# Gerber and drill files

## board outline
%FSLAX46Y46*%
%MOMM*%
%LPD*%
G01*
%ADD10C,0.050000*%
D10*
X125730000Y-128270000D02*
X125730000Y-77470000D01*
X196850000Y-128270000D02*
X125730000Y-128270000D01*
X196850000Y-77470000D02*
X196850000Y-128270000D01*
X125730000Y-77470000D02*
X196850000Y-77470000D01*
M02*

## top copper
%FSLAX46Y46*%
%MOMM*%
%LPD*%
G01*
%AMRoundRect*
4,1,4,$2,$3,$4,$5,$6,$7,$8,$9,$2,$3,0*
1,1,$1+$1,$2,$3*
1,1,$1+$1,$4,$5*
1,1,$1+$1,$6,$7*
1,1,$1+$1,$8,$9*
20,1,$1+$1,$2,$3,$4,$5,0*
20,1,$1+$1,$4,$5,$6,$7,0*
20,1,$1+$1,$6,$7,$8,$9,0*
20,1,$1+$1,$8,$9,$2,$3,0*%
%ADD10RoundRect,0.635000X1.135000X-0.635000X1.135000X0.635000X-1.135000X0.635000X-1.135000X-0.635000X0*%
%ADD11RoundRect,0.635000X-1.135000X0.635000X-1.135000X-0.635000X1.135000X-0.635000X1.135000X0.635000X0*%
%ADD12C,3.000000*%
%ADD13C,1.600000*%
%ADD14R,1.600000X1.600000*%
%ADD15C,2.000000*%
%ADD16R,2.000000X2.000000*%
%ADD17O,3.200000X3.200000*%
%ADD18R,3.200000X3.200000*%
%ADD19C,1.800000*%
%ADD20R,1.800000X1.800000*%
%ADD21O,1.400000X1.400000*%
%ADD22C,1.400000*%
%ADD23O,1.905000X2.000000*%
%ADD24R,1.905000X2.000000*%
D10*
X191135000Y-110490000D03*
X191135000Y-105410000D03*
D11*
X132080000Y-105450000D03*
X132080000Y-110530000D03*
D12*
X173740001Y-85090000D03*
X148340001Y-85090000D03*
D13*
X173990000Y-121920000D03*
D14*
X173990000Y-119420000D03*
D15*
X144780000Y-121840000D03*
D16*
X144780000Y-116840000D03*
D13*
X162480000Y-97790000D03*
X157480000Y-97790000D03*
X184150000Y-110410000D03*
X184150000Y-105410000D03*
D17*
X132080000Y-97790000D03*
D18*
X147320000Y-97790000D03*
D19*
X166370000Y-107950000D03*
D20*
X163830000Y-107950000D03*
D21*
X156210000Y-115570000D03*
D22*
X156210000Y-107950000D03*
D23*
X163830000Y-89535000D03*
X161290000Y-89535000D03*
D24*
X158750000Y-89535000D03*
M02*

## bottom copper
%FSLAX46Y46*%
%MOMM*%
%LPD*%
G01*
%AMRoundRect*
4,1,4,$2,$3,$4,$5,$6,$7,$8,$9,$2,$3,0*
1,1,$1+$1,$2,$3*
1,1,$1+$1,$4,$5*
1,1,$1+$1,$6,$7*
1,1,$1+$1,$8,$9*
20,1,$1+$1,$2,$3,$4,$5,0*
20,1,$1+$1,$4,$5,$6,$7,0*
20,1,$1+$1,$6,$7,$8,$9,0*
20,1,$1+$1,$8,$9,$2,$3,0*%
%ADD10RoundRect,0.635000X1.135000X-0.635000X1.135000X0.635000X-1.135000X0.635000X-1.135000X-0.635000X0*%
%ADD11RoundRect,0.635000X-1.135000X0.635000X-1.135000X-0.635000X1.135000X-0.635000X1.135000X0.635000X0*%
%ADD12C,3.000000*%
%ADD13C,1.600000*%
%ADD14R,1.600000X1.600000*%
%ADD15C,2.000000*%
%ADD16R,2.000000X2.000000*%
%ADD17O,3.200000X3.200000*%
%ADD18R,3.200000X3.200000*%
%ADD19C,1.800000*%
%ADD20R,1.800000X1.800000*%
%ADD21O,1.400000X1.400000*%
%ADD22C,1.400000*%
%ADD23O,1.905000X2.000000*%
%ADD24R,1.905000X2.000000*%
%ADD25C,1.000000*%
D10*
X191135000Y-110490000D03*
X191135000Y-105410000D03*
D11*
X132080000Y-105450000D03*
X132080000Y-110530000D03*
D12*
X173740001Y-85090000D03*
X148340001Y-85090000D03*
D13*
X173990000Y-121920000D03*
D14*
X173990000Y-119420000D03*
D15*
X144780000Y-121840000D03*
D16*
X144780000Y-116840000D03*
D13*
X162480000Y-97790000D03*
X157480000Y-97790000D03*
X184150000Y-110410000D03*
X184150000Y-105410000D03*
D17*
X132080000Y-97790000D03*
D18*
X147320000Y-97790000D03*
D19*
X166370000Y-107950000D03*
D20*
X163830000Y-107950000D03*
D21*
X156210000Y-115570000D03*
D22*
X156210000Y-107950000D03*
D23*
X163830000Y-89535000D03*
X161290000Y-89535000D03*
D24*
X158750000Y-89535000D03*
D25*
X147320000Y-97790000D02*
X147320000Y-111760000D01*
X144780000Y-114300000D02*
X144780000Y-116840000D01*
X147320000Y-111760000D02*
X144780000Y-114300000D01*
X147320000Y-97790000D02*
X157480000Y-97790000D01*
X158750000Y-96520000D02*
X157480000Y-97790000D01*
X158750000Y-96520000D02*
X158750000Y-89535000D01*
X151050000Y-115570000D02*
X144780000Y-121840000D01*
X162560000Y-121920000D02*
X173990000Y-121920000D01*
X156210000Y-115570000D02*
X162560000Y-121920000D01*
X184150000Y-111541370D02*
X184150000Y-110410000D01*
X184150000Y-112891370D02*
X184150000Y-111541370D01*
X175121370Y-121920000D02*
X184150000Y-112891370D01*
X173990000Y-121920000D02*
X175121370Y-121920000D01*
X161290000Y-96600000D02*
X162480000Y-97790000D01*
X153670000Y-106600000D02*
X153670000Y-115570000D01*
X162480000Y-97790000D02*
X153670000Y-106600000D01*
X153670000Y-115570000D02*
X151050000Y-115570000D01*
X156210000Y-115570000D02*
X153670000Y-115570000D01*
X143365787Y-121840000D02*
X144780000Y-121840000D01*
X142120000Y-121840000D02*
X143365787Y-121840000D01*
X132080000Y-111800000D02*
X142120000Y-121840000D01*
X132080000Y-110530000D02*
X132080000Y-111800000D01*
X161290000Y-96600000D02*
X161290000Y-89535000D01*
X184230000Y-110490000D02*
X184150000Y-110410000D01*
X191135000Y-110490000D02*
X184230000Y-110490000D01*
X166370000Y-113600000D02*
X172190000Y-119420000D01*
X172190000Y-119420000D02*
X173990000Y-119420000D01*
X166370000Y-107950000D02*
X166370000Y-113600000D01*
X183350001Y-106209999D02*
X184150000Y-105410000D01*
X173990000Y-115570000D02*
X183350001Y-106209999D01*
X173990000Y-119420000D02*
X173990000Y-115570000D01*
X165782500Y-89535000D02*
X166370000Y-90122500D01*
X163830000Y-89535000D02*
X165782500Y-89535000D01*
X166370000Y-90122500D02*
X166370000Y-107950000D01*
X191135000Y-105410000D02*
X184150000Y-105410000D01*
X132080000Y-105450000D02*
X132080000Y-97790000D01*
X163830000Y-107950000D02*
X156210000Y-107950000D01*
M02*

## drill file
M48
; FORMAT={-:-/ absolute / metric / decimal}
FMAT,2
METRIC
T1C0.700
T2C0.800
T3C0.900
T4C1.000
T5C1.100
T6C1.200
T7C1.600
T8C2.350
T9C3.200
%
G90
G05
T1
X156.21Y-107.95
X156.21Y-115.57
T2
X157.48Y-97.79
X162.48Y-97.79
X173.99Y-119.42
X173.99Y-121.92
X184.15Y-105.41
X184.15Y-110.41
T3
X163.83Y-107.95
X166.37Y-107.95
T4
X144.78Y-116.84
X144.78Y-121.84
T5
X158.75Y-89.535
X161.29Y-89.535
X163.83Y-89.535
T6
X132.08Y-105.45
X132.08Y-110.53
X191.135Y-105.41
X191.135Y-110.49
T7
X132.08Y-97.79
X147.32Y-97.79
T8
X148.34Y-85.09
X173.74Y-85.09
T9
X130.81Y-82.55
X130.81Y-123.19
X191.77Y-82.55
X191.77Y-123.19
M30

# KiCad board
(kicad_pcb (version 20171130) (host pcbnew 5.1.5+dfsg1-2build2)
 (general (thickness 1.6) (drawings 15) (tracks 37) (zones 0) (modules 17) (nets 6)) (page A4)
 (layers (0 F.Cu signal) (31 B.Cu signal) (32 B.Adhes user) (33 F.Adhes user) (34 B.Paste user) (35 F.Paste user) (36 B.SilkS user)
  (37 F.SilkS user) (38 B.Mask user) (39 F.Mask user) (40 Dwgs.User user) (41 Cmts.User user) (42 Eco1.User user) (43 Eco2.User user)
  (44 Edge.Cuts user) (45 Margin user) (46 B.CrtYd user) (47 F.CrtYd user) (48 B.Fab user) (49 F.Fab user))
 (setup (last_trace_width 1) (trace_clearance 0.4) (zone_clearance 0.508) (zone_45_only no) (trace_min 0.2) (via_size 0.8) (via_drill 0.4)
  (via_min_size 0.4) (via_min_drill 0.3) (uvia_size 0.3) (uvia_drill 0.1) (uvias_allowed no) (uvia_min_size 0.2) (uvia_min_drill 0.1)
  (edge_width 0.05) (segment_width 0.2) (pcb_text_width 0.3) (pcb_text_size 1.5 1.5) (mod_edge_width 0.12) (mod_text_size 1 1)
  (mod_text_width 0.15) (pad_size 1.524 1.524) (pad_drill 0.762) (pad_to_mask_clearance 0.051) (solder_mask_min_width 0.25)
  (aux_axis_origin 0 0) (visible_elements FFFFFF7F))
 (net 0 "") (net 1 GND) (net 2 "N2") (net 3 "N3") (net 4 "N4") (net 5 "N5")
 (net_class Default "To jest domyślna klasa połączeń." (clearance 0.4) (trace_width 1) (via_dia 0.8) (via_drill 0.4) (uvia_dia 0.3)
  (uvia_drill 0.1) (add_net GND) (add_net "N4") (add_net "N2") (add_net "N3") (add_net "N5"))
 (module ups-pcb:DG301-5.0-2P (layer F.Cu) (at 191.135 107.99 90)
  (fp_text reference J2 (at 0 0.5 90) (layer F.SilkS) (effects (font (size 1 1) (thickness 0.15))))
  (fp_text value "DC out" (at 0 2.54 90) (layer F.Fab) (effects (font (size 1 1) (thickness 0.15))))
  (pad 1 thru_hole roundrect (at -2.5 0 90) (size 2.54 3.54) (drill 1.2) (layers *.Cu *.Mask) (roundrect_rratio 0.25) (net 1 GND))
  (pad 2 thru_hole roundrect (at 2.58 0 90) (size 2.54 3.54) (drill 1.2) (layers *.Cu *.Mask) (roundrect_rratio 0.25) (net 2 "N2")))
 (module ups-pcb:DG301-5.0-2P (layer F.Cu) (at 132.08 107.95 270)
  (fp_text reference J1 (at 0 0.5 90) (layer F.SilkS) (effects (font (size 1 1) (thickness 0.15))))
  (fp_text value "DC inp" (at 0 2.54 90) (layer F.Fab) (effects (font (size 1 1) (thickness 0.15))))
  (pad 1 thru_hole roundrect (at -2.5 0 270) (size 2.54 3.54) (drill 1.2) (layers *.Cu *.Mask) (roundrect_rratio 0.25) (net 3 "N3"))
  (pad 2 thru_hole roundrect (at 2.58 0 270) (size 2.54 3.54) (drill 1.2) (layers *.Cu *.Mask) (roundrect_rratio 0.25) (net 1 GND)))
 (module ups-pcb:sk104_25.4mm (layer F.Cu) (at 161.040001 85.09)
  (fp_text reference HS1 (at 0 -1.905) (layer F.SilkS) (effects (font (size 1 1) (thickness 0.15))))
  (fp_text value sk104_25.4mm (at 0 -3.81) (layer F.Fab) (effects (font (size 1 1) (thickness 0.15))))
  (pad "" np_thru_hole circle (at 12.7 0) (size 3 3) (drill 2.35) (layers *.Cu *.Mask))
  (pad "" np_thru_hole circle (at -12.7 0) (size 3 3) (drill 2.35) (layers *.Cu *.Mask)))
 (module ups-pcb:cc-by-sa (layer F.Cu) (at 159.385 121.92)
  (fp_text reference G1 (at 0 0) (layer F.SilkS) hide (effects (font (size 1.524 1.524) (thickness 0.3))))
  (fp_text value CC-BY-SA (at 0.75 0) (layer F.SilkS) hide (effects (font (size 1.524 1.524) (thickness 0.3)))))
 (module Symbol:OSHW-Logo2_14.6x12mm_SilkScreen (layer F.Cu) (at 186.055 93.98)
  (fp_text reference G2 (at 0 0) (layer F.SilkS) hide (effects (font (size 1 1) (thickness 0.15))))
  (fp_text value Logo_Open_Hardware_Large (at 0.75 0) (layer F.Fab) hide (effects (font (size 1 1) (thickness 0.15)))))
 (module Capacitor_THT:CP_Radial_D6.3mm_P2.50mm (layer F.Cu) (at 173.99 119.42 270)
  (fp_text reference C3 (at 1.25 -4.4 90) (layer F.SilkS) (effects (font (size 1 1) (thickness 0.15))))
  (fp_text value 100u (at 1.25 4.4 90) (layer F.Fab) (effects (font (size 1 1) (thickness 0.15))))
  (pad 2 thru_hole circle (at 2.5 0 270) (size 1.6 1.6) (drill 0.8) (layers *.Cu *.Mask) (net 1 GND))
  (pad 1 thru_hole rect (at 0 0 270) (size 1.6 1.6) (drill 0.8) (layers *.Cu *.Mask) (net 2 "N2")))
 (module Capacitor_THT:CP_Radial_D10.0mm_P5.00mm (layer F.Cu) (at 144.78 116.84 270)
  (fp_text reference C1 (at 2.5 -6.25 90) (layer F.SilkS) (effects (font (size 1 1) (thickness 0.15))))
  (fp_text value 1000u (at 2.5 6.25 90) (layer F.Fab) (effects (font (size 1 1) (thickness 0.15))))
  (pad 2 thru_hole circle (at 5 0 270) (size 2 2) (drill 1) (layers *.Cu *.Mask) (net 1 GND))
  (pad 1 thru_hole rect (at 0 0 270) (size 2 2) (drill 1) (layers *.Cu *.Mask) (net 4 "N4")))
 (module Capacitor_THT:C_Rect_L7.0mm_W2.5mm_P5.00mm (layer F.Cu) (at 157.48 97.79)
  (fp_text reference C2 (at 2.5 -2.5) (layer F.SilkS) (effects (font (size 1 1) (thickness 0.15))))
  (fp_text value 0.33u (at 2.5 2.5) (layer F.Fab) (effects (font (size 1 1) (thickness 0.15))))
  (pad 2 thru_hole circle (at 5 0) (size 1.6 1.6) (drill 0.8) (layers *.Cu *.Mask) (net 1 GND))
  (pad 1 thru_hole circle (at 0 0) (size 1.6 1.6) (drill 0.8) (layers *.Cu *.Mask) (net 4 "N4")))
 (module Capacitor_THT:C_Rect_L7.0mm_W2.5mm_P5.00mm (layer F.Cu) (at 184.15 105.41 270)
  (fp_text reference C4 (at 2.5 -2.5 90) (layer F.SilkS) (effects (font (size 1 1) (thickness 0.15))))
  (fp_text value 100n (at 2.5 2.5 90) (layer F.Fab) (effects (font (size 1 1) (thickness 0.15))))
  (pad 2 thru_hole circle (at 5 0 270) (size 1.6 1.6) (drill 0.8) (layers *.Cu *.Mask) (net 1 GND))
  (pad 1 thru_hole circle (at 0 0 270) (size 1.6 1.6) (drill 0.8) (layers *.Cu *.Mask) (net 2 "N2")))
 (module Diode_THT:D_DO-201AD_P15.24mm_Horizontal (layer F.Cu) (at 147.32 97.79 180)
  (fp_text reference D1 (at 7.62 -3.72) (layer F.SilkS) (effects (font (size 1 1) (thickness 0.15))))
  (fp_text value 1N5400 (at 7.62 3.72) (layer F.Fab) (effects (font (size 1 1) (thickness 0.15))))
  (pad 2 thru_hole oval (at 15.24 0 180) (size 3.2 3.2) (drill 1.6) (layers *.Cu *.Mask) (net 3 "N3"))
  (pad 1 thru_hole rect (at 0 0 180) (size 3.2 3.2) (drill 1.6) (layers *.Cu *.Mask) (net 4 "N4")))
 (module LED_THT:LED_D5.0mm (layer F.Cu) (at 163.83 107.95)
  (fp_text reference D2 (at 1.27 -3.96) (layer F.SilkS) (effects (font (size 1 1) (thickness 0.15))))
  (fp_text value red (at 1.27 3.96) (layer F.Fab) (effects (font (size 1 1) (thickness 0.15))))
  (pad 2 thru_hole circle (at 2.54 0) (size 1.8 1.8) (drill 0.9) (layers *.Cu *.Mask) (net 2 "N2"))
  (pad 1 thru_hole rect (at 0 0) (size 1.8 1.8) (drill 0.9) (layers *.Cu *.Mask) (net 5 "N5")))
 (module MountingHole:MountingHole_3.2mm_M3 (layer F.Cu) (at 130.81 82.55)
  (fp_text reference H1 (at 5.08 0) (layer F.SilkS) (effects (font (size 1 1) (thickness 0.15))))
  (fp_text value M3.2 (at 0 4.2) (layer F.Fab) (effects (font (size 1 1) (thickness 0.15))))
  (pad 1 np_thru_hole circle (at 0 0) (size 3.2 3.2) (drill 3.2) (layers *.Cu *.Mask)))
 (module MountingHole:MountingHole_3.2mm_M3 (layer F.Cu) (at 191.77 82.55)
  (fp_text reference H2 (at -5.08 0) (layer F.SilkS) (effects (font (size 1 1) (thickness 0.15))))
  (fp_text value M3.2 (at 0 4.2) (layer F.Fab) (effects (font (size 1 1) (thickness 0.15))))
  (pad 1 np_thru_hole circle (at 0 0) (size 3.2 3.2) (drill 3.2) (layers *.Cu *.Mask)))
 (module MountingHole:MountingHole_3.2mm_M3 (layer F.Cu) (at 191.77 123.19)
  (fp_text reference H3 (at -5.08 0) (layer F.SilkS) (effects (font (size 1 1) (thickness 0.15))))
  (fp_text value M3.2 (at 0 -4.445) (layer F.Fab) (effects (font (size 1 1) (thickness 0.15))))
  (pad 1 np_thru_hole circle (at 0 0) (size 3.2 3.2) (drill 3.2) (layers *.Cu *.Mask)))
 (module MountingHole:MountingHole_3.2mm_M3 (layer F.Cu) (at 130.81 123.19)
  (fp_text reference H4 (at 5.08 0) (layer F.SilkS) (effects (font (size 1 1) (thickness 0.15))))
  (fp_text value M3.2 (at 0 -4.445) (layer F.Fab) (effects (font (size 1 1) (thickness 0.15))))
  (pad 1 np_thru_hole circle (at 0 0) (size 3.2 3.2) (drill 3.2) (layers *.Cu *.Mask)))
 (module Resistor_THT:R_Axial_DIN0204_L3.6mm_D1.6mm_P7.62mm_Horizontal (layer F.Cu) (at 156.21 107.95 270)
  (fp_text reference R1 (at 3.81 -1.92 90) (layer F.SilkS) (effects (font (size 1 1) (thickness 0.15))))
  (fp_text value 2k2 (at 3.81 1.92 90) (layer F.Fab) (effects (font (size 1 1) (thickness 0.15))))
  (pad 2 thru_hole oval (at 7.62 0 270) (size 1.4 1.4) (drill 0.7) (layers *.Cu *.Mask) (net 1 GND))
  (pad 1 thru_hole circle (at 0 0 270) (size 1.4 1.4) (drill 0.7) (layers *.Cu *.Mask) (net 5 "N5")))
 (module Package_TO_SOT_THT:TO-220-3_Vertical (layer F.Cu) (at 158.75 89.535)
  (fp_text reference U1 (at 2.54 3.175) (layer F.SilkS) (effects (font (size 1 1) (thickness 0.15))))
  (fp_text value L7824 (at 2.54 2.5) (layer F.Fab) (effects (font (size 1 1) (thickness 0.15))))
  (pad 3 thru_hole oval (at 5.08 0) (size 1.905 2) (drill 1.1) (layers *.Cu *.Mask) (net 2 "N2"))
  (pad 2 thru_hole oval (at 2.54 0) (size 1.905 2) (drill 1.1) (layers *.Cu *.Mask) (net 1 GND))
  (pad 1 thru_hole rect (at 0 0) (size 1.905 2) (drill 1.1) (layers *.Cu *.Mask) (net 4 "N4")))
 (gr_line (start 125.73 128.27) (end 125.73 77.47) (layer Edge.Cuts) (width 0.05))
 (gr_line (start 196.85 128.27) (end 125.73 128.27) (layer Edge.Cuts) (width 0.05))
 (gr_line (start 196.85 77.47) (end 196.85 128.27) (layer Edge.Cuts) (width 0.05))
 (gr_line (start 125.73 77.47) (end 196.85 77.47) (layer Edge.Cuts) (width 0.05))
 (segment (start 147.32 97.79) (end 147.32 111.76) (width 1) (layer B.Cu) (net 4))
 (segment (start 144.78 114.3) (end 144.78 116.84) (width 1) (layer B.Cu) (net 4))
 (segment (start 147.32 111.76) (end 144.78 114.3) (width 1) (layer B.Cu) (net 4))
 (segment (start 147.32 97.79) (end 157.48 97.79) (width 1) (layer B.Cu) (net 4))
 (segment (start 158.75 96.52) (end 157.48 97.79) (width 1) (layer B.Cu) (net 4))
 (segment (start 158.75 96.52) (end 158.75 89.535) (width 1) (layer B.Cu) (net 4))
 (segment (start 151.05 115.57) (end 144.78 121.84) (width 1) (layer B.Cu) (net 1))
 (segment (start 162.56 121.92) (end 173.99 121.92) (width 1) (layer B.Cu) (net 1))
 (segment (start 156.21 115.57) (end 162.56 121.92) (width 1) (layer B.Cu) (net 1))
 (segment (start 184.15 111.54137) (end 184.15 110.41) (width 1) (layer B.Cu) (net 1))
 (segment (start 184.15 112.89137) (end 184.15 111.54137) (width 1) (layer B.Cu) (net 1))
 (segment (start 175.12137 121.92) (end 184.15 112.89137) (width 1) (layer B.Cu) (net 1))
 (segment (start 173.99 121.92) (end 175.12137 121.92) (width 1) (layer B.Cu) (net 1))
 (segment (start 161.29 96.6) (end 162.48 97.79) (width 1) (layer B.Cu) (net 1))
 (segment (start 153.67 106.6) (end 153.67 115.57) (width 1) (layer B.Cu) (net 1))
 (segment (start 162.48 97.79) (end 153.67 106.6) (width 1) (layer B.Cu) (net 1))
 (segment (start 153.67 115.57) (end 151.05 115.57) (width 1) (layer B.Cu) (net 1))
 (segment (start 156.21 115.57) (end 153.67 115.57) (width 1) (layer B.Cu) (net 1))
 (segment (start 143.365787 121.84) (end 144.78 121.84) (width 1) (layer B.Cu) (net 1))
 (segment (start 142.12 121.84) (end 143.365787 121.84) (width 1) (layer B.Cu) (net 1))
 (segment (start 132.08 111.8) (end 142.12 121.84) (width 1) (layer B.Cu) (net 1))
 (segment (start 132.08 110.53) (end 132.08 111.8) (width 1) (layer B.Cu) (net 1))
 (segment (start 161.29 96.6) (end 161.29 89.535) (width 1) (layer B.Cu) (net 1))
 (segment (start 184.23 110.49) (end 184.15 110.41) (width 1) (layer B.Cu) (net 1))
 (segment (start 191.135 110.49) (end 184.23 110.49) (width 1) (layer B.Cu) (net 1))
 (segment (start 166.37 113.6) (end 172.19 119.42) (width 1) (layer B.Cu) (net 2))
 (segment (start 172.19 119.42) (end 173.99 119.42) (width 1) (layer B.Cu) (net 2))
 (segment (start 166.37 107.95) (end 166.37 113.6) (width 1) (layer B.Cu) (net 2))
 (segment (start 183.350001 106.209999) (end 184.15 105.41) (width 1) (layer B.Cu) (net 2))
 (segment (start 173.99 115.57) (end 183.350001 106.209999) (width 1) (layer B.Cu) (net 2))
 (segment (start 173.99 119.42) (end 173.99 115.57) (width 1) (layer B.Cu) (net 2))
 (segment (start 165.7825 89.535) (end 166.37 90.1225) (width 1) (layer B.Cu) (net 2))
 (segment (start 163.83 89.535) (end 165.7825 89.535) (width 1) (layer B.Cu) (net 2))
 (segment (start 166.37 90.1225) (end 166.37 107.95) (width 1) (layer B.Cu) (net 2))
 (segment (start 191.135 105.41) (end 184.15 105.41) (width 1) (layer B.Cu) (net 2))
 (segment (start 132.08 105.45) (end 132.08 97.79) (width 1) (layer B.Cu) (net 3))
 (segment (start 163.83 107.95) (end 156.21 107.95) (width 1) (layer B.Cu) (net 5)))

